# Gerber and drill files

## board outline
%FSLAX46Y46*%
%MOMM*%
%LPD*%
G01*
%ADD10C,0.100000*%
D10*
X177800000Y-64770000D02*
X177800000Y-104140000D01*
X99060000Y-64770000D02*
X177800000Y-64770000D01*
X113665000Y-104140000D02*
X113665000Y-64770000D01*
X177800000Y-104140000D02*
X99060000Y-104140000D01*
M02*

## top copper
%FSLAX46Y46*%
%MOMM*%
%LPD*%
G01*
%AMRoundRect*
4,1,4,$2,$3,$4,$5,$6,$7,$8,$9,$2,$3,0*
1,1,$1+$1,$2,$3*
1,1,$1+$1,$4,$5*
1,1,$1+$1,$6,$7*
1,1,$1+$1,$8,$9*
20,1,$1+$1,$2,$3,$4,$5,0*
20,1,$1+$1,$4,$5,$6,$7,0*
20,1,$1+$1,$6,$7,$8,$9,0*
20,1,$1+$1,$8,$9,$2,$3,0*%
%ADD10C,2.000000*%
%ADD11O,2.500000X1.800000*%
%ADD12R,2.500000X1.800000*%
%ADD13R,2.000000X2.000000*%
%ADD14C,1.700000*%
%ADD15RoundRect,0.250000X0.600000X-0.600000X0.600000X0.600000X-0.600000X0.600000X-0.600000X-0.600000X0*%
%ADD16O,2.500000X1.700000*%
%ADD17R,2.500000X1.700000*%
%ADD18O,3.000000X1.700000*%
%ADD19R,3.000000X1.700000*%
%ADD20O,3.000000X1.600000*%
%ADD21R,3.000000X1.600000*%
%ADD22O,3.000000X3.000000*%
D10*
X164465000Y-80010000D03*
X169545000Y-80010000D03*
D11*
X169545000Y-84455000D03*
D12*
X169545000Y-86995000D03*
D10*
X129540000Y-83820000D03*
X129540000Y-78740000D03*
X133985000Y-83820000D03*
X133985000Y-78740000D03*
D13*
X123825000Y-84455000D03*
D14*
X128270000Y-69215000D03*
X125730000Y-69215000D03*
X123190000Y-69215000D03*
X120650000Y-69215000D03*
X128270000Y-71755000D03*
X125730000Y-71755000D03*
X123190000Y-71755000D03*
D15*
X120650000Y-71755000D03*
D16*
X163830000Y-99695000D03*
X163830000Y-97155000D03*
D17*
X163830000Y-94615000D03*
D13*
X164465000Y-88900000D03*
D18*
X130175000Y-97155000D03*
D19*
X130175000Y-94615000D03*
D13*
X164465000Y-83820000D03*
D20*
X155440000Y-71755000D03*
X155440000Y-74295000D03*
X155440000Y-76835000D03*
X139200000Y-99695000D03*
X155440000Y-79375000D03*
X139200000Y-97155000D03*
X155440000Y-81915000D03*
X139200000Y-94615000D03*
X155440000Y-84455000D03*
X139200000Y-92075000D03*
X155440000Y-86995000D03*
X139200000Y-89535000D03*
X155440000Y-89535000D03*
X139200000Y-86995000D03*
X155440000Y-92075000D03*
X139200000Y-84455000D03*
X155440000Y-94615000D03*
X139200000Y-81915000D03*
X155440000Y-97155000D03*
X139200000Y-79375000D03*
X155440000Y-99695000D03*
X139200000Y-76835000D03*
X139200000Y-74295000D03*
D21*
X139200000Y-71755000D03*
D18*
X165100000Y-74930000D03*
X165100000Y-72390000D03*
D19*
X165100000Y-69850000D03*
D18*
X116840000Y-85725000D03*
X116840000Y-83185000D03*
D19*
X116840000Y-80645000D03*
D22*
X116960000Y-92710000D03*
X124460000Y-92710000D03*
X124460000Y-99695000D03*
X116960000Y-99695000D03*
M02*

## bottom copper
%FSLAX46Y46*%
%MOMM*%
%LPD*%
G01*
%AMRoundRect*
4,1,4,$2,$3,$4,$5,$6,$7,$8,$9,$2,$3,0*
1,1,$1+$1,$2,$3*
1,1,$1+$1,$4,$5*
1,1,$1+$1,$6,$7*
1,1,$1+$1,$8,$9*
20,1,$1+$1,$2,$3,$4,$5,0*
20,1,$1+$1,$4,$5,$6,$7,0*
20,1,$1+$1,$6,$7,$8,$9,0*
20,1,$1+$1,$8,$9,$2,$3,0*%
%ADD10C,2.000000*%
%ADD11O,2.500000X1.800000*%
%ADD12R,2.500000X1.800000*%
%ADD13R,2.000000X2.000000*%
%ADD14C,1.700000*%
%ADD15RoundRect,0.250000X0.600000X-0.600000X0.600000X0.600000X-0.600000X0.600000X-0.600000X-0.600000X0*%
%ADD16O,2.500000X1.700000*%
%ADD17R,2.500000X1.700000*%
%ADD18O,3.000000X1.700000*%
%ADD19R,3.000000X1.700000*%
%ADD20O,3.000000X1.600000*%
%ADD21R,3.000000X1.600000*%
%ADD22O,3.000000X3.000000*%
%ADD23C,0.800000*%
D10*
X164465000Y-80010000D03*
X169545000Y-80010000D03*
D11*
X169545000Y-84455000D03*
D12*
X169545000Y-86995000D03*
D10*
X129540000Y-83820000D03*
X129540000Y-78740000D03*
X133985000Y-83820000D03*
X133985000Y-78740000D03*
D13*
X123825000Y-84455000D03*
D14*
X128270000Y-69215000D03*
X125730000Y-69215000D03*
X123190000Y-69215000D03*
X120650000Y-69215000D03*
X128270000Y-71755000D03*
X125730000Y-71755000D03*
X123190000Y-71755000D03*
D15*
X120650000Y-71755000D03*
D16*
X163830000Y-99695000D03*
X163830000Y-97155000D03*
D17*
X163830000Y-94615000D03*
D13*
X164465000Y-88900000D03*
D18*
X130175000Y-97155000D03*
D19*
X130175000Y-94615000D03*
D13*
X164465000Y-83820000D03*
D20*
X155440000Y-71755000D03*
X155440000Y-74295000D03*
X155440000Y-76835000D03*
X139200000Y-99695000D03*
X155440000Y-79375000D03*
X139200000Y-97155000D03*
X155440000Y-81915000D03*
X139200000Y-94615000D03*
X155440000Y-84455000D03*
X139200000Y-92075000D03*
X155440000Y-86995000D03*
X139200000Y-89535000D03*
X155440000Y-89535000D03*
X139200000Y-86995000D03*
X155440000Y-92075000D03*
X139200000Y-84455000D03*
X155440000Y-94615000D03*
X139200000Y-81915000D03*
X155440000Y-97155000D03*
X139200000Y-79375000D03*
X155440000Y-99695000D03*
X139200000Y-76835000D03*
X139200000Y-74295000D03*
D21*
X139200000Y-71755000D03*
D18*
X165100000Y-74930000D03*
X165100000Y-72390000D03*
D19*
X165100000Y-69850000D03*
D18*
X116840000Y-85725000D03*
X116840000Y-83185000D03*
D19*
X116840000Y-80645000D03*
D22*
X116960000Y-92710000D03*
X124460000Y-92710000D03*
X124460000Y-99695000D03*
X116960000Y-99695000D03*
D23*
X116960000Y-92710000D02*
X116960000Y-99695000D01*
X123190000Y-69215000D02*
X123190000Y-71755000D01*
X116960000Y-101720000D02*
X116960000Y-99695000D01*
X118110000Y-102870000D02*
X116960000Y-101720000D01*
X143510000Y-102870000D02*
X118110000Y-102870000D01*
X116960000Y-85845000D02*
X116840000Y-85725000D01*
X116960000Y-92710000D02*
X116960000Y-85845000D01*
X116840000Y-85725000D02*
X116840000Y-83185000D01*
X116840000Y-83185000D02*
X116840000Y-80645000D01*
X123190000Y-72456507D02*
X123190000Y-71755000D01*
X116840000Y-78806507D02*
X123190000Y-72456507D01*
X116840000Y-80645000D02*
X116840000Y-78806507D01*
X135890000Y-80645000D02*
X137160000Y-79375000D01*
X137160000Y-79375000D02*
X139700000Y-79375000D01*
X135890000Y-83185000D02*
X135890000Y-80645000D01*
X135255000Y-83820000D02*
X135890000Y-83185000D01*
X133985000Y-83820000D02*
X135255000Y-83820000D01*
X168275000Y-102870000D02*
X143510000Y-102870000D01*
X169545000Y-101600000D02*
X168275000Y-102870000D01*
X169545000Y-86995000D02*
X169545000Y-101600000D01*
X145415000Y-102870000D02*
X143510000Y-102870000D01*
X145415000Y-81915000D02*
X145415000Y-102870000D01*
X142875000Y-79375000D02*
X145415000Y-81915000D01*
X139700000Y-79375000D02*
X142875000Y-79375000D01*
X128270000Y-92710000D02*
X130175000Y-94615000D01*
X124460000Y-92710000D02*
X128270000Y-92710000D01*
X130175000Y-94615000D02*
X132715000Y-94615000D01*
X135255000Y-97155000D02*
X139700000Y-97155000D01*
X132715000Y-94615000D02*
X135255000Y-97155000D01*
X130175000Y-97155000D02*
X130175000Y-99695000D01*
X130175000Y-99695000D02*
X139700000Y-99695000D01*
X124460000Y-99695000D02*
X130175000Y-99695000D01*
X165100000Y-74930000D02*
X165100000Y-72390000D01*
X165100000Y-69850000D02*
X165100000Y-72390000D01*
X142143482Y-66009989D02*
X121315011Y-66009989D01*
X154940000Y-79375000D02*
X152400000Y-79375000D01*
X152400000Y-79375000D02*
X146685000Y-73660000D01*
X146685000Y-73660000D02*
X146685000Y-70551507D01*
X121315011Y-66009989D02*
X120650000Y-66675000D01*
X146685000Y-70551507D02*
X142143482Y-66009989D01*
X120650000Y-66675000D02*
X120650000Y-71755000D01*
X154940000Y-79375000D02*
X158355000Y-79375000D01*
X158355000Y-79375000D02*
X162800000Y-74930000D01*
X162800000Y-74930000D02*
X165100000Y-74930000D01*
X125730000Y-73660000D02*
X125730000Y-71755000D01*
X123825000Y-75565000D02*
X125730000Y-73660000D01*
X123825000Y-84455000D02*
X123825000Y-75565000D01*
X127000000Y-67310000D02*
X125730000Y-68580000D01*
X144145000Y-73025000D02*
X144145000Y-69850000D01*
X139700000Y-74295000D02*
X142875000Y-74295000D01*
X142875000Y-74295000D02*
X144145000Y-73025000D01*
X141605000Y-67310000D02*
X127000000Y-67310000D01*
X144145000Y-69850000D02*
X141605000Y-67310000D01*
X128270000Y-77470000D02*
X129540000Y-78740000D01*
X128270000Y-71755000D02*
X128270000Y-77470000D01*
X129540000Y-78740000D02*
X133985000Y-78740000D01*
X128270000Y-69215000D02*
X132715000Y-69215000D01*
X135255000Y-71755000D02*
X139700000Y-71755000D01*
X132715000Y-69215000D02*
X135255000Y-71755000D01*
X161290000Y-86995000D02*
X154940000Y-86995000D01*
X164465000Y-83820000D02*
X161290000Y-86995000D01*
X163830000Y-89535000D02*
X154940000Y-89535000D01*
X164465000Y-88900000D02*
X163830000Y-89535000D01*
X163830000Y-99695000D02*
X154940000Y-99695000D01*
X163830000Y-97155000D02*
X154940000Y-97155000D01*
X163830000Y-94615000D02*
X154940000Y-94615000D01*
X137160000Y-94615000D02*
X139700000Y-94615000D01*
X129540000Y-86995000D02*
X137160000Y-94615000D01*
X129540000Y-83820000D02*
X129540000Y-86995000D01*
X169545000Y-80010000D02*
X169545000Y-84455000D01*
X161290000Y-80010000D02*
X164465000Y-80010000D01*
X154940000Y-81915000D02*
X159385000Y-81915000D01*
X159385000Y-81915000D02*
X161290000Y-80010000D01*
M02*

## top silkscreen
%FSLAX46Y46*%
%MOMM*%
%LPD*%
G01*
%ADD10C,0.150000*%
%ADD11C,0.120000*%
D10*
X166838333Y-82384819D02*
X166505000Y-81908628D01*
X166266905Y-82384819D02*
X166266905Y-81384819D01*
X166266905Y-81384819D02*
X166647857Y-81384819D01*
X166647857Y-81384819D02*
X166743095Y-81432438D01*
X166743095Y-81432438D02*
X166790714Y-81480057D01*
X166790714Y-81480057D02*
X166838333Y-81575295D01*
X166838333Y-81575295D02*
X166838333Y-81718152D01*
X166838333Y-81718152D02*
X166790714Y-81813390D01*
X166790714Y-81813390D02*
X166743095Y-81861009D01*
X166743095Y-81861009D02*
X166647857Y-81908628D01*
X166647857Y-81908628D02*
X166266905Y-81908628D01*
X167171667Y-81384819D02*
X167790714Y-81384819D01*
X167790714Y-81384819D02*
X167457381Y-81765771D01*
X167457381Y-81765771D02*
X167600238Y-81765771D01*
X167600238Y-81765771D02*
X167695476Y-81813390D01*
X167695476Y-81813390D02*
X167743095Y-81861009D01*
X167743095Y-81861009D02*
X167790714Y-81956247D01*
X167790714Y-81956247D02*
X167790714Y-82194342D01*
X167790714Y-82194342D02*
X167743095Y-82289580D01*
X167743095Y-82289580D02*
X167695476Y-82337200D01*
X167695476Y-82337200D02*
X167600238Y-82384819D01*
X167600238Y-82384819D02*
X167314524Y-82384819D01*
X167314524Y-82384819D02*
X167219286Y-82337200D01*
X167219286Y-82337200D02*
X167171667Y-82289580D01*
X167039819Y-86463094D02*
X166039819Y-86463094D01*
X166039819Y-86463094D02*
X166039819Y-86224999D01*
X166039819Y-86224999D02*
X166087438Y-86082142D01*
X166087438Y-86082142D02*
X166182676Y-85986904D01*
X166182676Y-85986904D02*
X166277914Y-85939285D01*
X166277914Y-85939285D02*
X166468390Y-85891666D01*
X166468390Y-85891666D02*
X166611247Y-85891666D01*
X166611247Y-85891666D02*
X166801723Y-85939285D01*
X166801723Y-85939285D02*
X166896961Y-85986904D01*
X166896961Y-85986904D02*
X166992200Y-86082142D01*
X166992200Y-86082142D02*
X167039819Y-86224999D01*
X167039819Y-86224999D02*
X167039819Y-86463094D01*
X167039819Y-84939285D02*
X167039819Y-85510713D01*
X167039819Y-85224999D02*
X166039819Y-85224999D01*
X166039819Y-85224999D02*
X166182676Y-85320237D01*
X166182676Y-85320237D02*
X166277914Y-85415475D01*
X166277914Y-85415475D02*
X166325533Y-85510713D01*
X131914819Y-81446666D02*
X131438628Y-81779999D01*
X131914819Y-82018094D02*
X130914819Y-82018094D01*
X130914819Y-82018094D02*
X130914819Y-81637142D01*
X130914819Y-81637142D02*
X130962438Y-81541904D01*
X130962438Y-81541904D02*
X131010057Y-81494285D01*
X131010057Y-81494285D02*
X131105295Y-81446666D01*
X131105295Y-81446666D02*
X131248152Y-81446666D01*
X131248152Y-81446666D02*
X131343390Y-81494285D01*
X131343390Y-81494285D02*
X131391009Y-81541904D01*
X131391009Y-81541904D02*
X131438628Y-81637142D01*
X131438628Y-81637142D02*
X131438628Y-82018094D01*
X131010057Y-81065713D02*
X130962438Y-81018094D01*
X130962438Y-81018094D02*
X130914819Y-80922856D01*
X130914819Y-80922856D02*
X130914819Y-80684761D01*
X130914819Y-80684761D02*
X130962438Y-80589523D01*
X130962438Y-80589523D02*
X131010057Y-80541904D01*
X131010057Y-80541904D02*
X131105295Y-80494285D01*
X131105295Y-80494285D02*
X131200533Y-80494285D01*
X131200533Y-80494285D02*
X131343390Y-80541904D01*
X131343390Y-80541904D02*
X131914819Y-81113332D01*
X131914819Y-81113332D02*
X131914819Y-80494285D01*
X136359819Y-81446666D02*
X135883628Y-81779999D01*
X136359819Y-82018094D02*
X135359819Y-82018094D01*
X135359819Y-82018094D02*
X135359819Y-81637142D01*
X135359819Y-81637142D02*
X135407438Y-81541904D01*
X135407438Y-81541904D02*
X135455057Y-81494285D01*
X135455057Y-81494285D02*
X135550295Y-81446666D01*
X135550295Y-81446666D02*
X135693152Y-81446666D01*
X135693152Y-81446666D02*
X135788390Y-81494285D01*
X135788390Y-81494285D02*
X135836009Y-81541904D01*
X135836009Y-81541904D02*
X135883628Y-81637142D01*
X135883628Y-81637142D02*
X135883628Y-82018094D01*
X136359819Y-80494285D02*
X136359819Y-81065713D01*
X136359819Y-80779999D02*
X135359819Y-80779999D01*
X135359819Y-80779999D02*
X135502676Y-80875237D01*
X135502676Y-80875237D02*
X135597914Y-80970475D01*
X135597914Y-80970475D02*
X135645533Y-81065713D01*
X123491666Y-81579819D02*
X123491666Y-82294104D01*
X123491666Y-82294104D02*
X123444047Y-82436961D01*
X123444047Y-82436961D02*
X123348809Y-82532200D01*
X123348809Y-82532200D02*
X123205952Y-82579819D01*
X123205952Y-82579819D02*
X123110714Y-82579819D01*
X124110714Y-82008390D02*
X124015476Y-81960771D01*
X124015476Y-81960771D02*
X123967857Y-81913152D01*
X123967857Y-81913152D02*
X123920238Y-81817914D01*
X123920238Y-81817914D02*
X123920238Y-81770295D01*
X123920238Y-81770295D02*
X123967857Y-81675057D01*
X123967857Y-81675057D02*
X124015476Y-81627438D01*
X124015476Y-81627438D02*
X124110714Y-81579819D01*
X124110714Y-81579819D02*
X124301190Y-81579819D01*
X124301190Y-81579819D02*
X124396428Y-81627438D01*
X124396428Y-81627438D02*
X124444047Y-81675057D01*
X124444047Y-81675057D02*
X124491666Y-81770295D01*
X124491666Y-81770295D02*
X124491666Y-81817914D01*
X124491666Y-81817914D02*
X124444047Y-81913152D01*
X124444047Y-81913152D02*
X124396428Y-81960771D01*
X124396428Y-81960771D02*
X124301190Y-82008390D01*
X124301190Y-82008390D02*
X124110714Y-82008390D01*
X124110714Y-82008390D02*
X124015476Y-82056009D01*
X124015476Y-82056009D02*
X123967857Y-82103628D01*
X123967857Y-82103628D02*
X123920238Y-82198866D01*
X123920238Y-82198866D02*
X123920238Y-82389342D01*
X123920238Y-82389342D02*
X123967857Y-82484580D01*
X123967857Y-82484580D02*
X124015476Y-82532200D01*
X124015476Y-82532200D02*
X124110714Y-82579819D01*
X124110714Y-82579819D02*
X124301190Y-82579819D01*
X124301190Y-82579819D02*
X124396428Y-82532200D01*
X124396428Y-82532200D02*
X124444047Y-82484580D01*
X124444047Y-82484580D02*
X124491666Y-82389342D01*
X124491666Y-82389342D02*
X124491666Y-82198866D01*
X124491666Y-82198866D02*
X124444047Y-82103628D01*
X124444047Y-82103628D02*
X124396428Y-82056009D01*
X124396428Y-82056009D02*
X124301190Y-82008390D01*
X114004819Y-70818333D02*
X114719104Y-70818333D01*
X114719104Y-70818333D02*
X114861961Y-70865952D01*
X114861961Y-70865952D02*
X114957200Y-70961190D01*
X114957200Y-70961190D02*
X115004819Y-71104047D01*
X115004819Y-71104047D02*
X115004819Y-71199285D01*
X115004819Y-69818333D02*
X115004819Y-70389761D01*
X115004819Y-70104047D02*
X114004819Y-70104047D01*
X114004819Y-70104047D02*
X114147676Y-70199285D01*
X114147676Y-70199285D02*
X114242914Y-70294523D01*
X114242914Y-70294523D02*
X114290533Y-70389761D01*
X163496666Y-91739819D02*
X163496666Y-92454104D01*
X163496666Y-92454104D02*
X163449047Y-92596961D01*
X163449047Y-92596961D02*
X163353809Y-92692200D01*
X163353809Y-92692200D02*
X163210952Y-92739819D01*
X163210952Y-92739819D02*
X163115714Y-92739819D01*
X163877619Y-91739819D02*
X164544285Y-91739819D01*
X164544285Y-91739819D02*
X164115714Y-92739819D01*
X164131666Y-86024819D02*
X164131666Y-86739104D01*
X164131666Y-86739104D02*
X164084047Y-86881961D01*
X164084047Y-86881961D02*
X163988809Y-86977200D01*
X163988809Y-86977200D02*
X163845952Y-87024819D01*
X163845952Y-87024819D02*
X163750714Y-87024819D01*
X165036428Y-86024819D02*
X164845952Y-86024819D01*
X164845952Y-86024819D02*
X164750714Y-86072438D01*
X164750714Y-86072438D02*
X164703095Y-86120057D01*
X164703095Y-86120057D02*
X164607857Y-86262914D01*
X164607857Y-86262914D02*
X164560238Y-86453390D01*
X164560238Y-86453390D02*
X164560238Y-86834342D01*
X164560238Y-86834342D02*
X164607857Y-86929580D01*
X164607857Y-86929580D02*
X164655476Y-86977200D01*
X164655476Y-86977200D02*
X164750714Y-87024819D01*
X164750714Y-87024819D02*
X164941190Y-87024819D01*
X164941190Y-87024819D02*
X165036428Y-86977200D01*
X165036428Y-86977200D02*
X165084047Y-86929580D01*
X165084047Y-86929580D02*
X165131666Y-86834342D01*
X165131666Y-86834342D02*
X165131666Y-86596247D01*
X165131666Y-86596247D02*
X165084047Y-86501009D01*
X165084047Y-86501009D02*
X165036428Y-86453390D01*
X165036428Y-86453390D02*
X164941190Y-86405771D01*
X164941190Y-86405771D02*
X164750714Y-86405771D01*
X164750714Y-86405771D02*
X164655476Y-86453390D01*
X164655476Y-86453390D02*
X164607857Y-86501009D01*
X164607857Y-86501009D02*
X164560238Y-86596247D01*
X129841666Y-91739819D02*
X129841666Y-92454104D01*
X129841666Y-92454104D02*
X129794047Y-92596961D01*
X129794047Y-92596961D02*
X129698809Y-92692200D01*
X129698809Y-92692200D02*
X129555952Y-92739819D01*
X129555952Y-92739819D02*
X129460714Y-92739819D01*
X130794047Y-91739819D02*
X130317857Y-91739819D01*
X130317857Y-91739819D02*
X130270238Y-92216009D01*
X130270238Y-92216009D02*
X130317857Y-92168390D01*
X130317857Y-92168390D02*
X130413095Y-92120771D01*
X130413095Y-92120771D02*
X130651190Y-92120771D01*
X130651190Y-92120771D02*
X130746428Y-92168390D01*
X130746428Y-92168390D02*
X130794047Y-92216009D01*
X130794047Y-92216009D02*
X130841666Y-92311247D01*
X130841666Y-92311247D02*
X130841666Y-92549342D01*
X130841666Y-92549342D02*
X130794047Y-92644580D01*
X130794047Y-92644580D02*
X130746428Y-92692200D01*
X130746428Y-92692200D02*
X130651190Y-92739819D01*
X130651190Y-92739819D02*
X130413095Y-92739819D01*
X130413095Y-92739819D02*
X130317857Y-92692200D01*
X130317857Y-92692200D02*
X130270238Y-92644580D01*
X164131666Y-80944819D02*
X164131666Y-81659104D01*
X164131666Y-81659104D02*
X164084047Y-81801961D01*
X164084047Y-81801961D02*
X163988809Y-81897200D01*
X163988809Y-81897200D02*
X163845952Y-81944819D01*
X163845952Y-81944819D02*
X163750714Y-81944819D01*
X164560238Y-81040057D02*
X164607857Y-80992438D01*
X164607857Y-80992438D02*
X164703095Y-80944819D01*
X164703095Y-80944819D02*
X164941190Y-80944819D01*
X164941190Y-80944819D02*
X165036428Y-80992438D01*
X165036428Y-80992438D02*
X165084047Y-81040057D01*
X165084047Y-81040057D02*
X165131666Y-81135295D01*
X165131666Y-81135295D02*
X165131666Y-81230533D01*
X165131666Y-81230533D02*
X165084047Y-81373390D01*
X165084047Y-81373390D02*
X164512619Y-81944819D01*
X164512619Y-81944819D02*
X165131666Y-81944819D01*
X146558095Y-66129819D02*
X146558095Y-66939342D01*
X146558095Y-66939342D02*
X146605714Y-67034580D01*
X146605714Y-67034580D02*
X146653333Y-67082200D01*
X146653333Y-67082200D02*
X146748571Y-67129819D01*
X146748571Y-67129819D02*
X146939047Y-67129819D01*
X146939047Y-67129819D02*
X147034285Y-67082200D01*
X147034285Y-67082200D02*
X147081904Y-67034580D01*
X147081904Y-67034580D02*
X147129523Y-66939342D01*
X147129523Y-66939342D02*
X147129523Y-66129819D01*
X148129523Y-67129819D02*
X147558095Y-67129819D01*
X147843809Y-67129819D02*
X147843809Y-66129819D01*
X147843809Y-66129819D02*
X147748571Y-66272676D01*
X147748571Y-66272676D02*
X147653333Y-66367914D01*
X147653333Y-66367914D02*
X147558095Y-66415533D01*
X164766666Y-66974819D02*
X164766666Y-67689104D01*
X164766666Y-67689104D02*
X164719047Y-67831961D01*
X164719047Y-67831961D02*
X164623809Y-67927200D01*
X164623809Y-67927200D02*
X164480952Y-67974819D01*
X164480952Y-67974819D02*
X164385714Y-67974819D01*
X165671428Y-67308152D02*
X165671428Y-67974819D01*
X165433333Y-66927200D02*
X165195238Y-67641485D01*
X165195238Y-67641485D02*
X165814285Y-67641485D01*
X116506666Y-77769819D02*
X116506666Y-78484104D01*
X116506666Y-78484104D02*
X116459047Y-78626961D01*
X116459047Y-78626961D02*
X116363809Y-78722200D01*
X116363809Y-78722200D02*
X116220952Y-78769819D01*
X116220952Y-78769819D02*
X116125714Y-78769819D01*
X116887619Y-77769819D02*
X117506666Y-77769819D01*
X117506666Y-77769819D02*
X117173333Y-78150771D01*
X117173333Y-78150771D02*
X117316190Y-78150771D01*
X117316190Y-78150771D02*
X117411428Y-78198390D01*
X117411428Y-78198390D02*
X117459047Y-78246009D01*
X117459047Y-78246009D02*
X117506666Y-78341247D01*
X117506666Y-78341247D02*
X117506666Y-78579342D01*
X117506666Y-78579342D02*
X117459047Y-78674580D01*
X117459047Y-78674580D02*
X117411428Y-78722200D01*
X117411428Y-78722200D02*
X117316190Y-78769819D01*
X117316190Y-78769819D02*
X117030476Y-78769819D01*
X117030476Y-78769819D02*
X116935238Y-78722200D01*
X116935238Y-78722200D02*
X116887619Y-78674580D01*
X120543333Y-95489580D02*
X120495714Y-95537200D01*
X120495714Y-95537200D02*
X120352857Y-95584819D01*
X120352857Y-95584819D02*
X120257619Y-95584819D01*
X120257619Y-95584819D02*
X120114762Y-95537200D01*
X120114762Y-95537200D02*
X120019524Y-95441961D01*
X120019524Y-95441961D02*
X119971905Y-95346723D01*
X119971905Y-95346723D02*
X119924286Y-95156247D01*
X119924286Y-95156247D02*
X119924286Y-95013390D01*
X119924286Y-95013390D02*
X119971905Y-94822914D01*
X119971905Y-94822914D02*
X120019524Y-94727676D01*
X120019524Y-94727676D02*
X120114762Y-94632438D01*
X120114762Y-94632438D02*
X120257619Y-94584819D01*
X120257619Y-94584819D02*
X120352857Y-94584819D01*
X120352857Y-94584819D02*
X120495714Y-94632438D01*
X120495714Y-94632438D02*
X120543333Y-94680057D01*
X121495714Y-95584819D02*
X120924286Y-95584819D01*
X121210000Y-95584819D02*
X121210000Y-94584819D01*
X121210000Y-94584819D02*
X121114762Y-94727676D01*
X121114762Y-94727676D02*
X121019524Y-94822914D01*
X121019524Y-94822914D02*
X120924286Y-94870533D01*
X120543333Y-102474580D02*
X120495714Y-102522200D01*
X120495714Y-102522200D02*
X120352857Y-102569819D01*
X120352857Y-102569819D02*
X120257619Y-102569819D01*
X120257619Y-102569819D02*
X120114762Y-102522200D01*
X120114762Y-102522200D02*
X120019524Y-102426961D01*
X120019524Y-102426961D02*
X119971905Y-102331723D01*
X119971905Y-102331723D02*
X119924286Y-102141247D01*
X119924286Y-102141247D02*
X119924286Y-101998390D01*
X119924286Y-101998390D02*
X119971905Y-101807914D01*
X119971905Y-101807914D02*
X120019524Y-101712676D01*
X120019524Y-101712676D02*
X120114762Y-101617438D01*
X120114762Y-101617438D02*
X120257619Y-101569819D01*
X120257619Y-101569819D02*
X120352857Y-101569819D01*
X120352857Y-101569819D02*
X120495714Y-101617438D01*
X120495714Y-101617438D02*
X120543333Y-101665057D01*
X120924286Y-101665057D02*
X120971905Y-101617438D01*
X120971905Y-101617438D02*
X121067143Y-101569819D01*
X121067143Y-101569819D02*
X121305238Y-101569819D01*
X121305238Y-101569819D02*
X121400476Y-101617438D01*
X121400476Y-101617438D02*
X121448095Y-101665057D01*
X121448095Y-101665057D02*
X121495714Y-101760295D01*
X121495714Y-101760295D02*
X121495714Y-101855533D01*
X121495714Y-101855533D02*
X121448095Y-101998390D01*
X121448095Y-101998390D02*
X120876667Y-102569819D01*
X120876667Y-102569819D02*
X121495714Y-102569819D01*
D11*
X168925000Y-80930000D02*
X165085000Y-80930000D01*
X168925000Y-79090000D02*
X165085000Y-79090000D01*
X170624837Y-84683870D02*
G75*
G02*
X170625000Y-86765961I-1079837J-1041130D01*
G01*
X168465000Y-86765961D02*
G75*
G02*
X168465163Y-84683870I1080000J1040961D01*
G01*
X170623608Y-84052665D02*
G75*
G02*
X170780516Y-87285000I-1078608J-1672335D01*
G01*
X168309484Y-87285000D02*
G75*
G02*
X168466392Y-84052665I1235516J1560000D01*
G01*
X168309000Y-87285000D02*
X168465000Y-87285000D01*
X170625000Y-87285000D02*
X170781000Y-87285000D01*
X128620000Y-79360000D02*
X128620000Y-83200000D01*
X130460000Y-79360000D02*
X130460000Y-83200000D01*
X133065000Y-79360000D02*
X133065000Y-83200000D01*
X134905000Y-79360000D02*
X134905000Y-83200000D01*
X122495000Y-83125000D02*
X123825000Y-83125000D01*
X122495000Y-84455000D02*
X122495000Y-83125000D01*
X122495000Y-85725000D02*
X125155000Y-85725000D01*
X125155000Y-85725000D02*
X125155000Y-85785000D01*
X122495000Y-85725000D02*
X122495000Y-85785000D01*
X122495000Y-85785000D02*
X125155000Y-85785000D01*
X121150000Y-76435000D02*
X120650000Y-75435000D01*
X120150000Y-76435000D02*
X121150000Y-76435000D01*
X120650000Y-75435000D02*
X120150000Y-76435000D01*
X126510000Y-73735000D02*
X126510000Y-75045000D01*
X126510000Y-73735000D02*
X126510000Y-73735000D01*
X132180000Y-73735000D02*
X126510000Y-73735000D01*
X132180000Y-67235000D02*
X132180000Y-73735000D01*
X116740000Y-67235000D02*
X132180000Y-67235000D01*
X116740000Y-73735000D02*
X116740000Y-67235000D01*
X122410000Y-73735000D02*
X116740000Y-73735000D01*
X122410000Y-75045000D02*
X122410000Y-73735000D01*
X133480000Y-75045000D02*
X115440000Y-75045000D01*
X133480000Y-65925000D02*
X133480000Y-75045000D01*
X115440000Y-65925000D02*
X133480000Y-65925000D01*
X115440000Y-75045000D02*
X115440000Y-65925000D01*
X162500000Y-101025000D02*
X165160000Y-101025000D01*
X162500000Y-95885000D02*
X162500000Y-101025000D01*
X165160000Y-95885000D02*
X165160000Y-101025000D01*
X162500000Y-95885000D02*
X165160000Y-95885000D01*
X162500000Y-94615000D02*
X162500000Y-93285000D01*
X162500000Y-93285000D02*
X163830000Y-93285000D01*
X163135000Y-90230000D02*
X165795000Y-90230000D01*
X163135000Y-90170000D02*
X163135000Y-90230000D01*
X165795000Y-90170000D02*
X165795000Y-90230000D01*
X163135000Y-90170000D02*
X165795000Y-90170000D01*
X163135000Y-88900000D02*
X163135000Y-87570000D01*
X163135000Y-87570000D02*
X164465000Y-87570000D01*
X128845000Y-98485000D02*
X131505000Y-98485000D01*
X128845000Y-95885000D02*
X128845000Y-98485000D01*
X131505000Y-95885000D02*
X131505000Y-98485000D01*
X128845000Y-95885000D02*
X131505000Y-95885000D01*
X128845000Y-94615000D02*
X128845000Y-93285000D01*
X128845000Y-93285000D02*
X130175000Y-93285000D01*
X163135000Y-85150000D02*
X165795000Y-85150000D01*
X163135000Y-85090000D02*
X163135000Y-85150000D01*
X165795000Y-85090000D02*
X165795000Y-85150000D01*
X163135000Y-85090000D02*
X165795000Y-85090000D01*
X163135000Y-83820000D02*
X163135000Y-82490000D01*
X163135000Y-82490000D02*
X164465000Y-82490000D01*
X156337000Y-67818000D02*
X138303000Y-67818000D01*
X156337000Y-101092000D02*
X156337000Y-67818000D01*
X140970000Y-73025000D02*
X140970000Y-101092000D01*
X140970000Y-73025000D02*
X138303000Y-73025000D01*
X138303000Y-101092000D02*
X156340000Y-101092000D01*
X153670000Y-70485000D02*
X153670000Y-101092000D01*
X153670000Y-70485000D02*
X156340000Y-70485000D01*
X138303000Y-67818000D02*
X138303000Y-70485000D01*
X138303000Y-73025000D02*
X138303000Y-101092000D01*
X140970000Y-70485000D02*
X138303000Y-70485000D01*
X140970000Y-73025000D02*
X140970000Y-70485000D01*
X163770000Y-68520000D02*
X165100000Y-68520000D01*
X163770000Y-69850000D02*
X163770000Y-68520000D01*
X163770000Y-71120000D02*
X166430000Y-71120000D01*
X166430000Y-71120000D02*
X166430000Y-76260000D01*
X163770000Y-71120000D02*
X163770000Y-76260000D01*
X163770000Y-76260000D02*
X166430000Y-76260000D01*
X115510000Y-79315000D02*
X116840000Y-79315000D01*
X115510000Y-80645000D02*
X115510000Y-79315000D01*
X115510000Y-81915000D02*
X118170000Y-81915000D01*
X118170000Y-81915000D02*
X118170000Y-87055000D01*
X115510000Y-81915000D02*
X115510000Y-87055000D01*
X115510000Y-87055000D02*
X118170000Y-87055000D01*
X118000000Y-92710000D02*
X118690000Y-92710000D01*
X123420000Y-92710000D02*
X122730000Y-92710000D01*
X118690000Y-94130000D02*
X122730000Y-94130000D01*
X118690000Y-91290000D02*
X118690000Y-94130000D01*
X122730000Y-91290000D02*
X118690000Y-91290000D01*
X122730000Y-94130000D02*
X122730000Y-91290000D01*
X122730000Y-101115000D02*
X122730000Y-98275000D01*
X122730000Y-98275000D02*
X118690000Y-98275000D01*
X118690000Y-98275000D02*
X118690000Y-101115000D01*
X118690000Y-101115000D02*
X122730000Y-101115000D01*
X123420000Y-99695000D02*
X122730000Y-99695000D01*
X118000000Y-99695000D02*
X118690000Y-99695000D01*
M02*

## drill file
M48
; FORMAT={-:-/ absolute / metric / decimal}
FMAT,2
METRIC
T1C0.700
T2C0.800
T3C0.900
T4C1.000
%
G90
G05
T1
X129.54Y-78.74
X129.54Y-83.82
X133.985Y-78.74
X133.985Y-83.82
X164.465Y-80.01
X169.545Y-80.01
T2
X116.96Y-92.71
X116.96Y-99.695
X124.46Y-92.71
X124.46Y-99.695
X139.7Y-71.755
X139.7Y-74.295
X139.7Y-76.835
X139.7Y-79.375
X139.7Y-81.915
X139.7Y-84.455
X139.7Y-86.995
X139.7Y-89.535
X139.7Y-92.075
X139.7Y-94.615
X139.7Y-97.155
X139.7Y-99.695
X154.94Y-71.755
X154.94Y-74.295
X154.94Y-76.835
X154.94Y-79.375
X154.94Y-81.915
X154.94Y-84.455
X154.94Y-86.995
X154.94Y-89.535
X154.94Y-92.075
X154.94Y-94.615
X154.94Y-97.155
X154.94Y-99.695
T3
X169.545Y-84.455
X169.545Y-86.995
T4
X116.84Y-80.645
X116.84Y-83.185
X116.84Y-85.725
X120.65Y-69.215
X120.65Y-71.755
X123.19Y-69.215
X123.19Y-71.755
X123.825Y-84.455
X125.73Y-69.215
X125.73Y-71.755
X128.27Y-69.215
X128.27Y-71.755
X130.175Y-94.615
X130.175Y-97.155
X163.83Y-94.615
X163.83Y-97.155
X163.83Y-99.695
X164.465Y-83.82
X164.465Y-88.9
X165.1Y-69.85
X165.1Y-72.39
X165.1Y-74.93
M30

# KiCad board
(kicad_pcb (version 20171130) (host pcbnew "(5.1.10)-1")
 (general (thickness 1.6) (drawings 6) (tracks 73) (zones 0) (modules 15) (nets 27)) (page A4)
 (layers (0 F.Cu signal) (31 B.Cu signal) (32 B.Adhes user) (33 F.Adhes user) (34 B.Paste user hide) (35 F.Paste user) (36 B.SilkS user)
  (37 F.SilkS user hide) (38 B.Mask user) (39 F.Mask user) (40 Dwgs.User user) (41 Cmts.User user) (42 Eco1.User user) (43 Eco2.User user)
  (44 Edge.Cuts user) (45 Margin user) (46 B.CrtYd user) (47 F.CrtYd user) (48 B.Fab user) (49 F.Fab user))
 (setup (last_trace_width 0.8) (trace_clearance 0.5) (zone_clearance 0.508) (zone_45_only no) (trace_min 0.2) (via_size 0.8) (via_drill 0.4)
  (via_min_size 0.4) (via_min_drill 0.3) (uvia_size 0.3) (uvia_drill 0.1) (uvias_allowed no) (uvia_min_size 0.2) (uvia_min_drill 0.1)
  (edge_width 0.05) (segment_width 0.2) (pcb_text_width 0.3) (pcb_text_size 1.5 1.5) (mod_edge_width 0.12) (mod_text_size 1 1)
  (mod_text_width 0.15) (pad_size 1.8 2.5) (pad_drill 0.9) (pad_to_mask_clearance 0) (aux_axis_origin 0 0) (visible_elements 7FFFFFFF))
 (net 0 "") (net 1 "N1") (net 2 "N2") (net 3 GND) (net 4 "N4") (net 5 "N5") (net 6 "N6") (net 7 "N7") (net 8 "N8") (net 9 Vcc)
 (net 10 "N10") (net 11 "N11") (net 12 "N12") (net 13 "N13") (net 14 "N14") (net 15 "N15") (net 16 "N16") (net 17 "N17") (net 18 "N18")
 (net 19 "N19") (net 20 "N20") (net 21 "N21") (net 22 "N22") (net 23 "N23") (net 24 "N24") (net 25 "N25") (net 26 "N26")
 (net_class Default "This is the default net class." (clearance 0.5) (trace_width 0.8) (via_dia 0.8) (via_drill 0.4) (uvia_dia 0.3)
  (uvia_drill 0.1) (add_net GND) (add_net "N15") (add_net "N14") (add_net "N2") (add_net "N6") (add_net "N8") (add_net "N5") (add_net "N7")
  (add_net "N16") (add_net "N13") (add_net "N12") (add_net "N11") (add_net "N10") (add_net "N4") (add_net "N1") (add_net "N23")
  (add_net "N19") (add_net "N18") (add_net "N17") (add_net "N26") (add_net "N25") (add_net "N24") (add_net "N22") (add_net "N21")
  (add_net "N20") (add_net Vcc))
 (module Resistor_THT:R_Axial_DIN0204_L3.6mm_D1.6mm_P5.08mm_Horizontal (layer F.Cu) (at 169.545 80.01 180)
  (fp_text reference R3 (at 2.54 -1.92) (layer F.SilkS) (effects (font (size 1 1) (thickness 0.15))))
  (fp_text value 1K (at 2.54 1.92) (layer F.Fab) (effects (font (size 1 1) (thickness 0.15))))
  (fp_line (start 0.62 -0.92) (end 4.46 -0.92) (layer F.SilkS) (width 0.12))
  (fp_line (start 0.62 0.92) (end 4.46 0.92) (layer F.SilkS) (width 0.12))
  (pad 2 thru_hole circle (at 5.08 0 180) (size 2 2) (drill 0.7) (layers *.Cu *.Mask) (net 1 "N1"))
  (pad 1 thru_hole circle (at 0 0 180) (size 2 2) (drill 0.7) (layers *.Cu *.Mask) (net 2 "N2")))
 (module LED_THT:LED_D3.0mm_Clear (layer F.Cu) (at 169.545 86.995 90)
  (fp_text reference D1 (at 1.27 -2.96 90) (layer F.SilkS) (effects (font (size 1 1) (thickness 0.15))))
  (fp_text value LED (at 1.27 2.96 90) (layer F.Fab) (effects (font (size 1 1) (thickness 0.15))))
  (fp_arc (start 1.27 0) (end 0.229039 1.08) (angle -87.9) (layer F.SilkS) (width 0.12))
  (fp_arc (start 1.27 0) (end 0.229039 -1.08) (angle 87.9) (layer F.SilkS) (width 0.12))
  (fp_arc (start 1.27 0) (end -0.29 1.235516) (angle -108.8) (layer F.SilkS) (width 0.12))
  (fp_arc (start 1.27 0) (end -0.29 -1.235516) (angle 108.8) (layer F.SilkS) (width 0.12))
  (fp_line (start -0.29 -1.236) (end -0.29 -1.08) (layer F.SilkS) (width 0.12))
  (fp_line (start -0.29 1.08) (end -0.29 1.236) (layer F.SilkS) (width 0.12))
  (pad 2 thru_hole oval (at 2.54 0 90) (size 1.8 2.5) (drill 0.9) (layers *.Cu *.Mask) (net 2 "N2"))
  (pad 1 thru_hole rect (at 0 0 90) (size 1.8 2.5) (drill 0.9) (layers *.Cu *.Mask) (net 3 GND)))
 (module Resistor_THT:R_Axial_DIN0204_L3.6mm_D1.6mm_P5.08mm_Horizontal (layer F.Cu) (at 129.54 78.74 270)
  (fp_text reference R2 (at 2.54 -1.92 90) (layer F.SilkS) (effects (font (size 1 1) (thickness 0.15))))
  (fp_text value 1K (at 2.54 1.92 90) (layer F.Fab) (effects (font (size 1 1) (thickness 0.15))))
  (fp_line (start 0.62 0.92) (end 4.46 0.92) (layer F.SilkS) (width 0.12))
  (fp_line (start 0.62 -0.92) (end 4.46 -0.92) (layer F.SilkS) (width 0.12))
  (pad 2 thru_hole circle (at 5.08 0 270) (size 2 2) (drill 0.7) (layers *.Cu *.Mask) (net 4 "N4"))
  (pad 1 thru_hole circle (at 0 0 270) (size 2 2) (drill 0.7) (layers *.Cu *.Mask) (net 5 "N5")))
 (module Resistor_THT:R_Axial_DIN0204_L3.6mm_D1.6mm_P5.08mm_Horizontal (layer F.Cu) (at 133.985 78.74 270)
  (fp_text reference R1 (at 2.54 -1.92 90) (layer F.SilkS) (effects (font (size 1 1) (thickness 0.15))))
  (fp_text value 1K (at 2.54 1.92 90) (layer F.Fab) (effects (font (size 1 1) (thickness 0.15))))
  (fp_line (start 0.62 0.92) (end 4.46 0.92) (layer F.SilkS) (width 0.12))
  (fp_line (start 0.62 -0.92) (end 4.46 -0.92) (layer F.SilkS) (width 0.12))
  (pad 2 thru_hole circle (at 5.08 0 270) (size 2 2) (drill 0.7) (layers *.Cu *.Mask) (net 3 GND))
  (pad 1 thru_hole circle (at 0 0 270) (size 2 2) (drill 0.7) (layers *.Cu *.Mask) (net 5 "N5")))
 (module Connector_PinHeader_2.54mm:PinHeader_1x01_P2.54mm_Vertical (layer F.Cu) (at 123.825 84.455)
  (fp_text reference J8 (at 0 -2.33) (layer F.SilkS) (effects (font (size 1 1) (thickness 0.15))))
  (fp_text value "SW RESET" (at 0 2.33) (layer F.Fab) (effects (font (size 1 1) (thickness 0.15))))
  (fp_line (start -1.33 -1.33) (end 0 -1.33) (layer F.SilkS) (width 0.12))
  (fp_line (start -1.33 0) (end -1.33 -1.33) (layer F.SilkS) (width 0.12))
  (fp_line (start -1.33 1.27) (end 1.33 1.27) (layer F.SilkS) (width 0.12))
  (fp_line (start 1.33 1.27) (end 1.33 1.33) (layer F.SilkS) (width 0.12))
  (fp_line (start -1.33 1.27) (end -1.33 1.33) (layer F.SilkS) (width 0.12))
  (fp_line (start -1.33 1.33) (end 1.33 1.33) (layer F.SilkS) (width 0.12))
  (pad 1 thru_hole rect (at 0 0) (size 2 2) (drill 1) (layers *.Cu *.Mask) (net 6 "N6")))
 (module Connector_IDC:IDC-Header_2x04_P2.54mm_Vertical (layer F.Cu) (at 120.65 71.755 90)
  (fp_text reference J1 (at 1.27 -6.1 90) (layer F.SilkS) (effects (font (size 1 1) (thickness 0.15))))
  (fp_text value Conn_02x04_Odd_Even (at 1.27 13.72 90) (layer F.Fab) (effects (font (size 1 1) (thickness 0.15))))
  (fp_line (start -4.68 0.5) (end -3.68 0) (layer F.SilkS) (width 0.12))
  (fp_line (start -4.68 -0.5) (end -4.68 0.5) (layer F.SilkS) (width 0.12))
  (fp_line (start -3.68 0) (end -4.68 -0.5) (layer F.SilkS) (width 0.12))
  (fp_line (start -1.98 5.86) (end -3.29 5.86) (layer F.SilkS) (width 0.12))
  (fp_line (start -1.98 5.86) (end -1.98 5.86) (layer F.SilkS) (width 0.12))
  (fp_line (start -1.98 11.53) (end -1.98 5.86) (layer F.SilkS) (width 0.12))
  (fp_line (start 4.52 11.53) (end -1.98 11.53) (layer F.SilkS) (width 0.12))
  (fp_line (start 4.52 -3.91) (end 4.52 11.53) (layer F.SilkS) (width 0.12))
  (fp_line (start -1.98 -3.91) (end 4.52 -3.91) (layer F.SilkS) (width 0.12))
  (fp_line (start -1.98 1.76) (end -1.98 -3.91) (layer F.SilkS) (width 0.12))
  (fp_line (start -3.29 1.76) (end -1.98 1.76) (layer F.SilkS) (width 0.12))
  (fp_line (start -3.29 12.83) (end -3.29 -5.21) (layer F.SilkS) (width 0.12))
  (fp_line (start 5.83 12.83) (end -3.29 12.83) (layer F.SilkS) (width 0.12))
  (fp_line (start 5.83 -5.21) (end 5.83 12.83) (layer F.SilkS) (width 0.12))
  (fp_line (start -3.29 -5.21) (end 5.83 -5.21) (layer F.SilkS) (width 0.12))
  (pad 8 thru_hole circle (at 2.54 7.62 90) (size 1.7 1.7) (drill 1) (layers *.Cu *.Mask) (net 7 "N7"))
  (pad 6 thru_hole circle (at 2.54 5.08 90) (size 1.7 1.7) (drill 1) (layers *.Cu *.Mask) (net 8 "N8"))
  (pad 4 thru_hole circle (at 2.54 2.54 90) (size 1.7 1.7) (drill 1) (layers *.Cu *.Mask) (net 3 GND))
  (pad 2 thru_hole circle (at 2.54 0 90) (size 1.7 1.7) (drill 1) (layers *.Cu *.Mask) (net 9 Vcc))
  (pad 7 thru_hole circle (at 0 7.62 90) (size 1.7 1.7) (drill 1) (layers *.Cu *.Mask) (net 5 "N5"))
  (pad 5 thru_hole circle (at 0 5.08 90) (size 1.7 1.7) (drill 1) (layers *.Cu *.Mask) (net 6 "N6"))
  (pad 3 thru_hole circle (at 0 2.54 90) (size 1.7 1.7) (drill 1) (layers *.Cu *.Mask) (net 3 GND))
  (pad 1 thru_hole roundrect (at 0 0 90) (size 1.7 1.7) (drill 1) (layers *.Cu *.Mask) (roundrect_rratio 0.147059) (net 9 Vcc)))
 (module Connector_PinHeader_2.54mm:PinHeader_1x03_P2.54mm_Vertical (layer F.Cu) (at 163.83 94.615)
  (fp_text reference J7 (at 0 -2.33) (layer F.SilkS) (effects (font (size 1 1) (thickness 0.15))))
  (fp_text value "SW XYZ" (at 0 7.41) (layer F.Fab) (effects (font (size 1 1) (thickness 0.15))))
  (fp_line (start -1.33 6.41) (end 1.33 6.41) (layer F.SilkS) (width 0.12))
  (fp_line (start -1.33 1.27) (end -1.33 6.41) (layer F.SilkS) (width 0.12))
  (fp_line (start 1.33 1.27) (end 1.33 6.41) (layer F.SilkS) (width 0.12))
  (fp_line (start -1.33 1.27) (end 1.33 1.27) (layer F.SilkS) (width 0.12))
  (fp_line (start -1.33 0) (end -1.33 -1.33) (layer F.SilkS) (width 0.12))
  (fp_line (start -1.33 -1.33) (end 0 -1.33) (layer F.SilkS) (width 0.12))
  (pad 3 thru_hole oval (at 0 5.08) (size 2.5 1.7) (drill 1) (layers *.Cu *.Mask) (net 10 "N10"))
  (pad 2 thru_hole oval (at 0 2.54) (size 2.5 1.7) (drill 1) (layers *.Cu *.Mask) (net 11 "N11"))
  (pad 1 thru_hole rect (at 0 0) (size 2.5 1.7) (drill 1) (layers *.Cu *.Mask) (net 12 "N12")))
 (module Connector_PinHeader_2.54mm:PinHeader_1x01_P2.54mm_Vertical (layer F.Cu) (at 164.465 88.9)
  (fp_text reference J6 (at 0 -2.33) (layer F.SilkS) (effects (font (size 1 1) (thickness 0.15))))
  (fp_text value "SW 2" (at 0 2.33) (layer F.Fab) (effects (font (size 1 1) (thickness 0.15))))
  (fp_line (start -1.33 1.33) (end 1.33 1.33) (layer F.SilkS) (width 0.12))
  (fp_line (start -1.33 1.27) (end -1.33 1.33) (layer F.SilkS) (width 0.12))
  (fp_line (start 1.33 1.27) (end 1.33 1.33) (layer F.SilkS) (width 0.12))
  (fp_line (start -1.33 1.27) (end 1.33 1.27) (layer F.SilkS) (width 0.12))
  (fp_line (start -1.33 0) (end -1.33 -1.33) (layer F.SilkS) (width 0.12))
  (fp_line (start -1.33 -1.33) (end 0 -1.33) (layer F.SilkS) (width 0.12))
  (pad 1 thru_hole rect (at 0 0) (size 2 2) (drill 1) (layers *.Cu *.Mask) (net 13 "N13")))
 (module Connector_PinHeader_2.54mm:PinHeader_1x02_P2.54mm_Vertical (layer F.Cu) (at 130.175 94.615)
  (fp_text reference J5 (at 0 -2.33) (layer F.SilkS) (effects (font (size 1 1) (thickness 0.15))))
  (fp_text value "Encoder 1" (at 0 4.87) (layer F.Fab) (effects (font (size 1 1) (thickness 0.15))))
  (fp_line (start -1.33 3.87) (end 1.33 3.87) (layer F.SilkS) (width 0.12))
  (fp_line (start -1.33 1.27) (end -1.33 3.87) (layer F.SilkS) (width 0.12))
  (fp_line (start 1.33 1.27) (end 1.33 3.87) (layer F.SilkS) (width 0.12))
  (fp_line (start -1.33 1.27) (end 1.33 1.27) (layer F.SilkS) (width 0.12))
  (fp_line (start -1.33 0) (end -1.33 -1.33) (layer F.SilkS) (width 0.12))
  (fp_line (start -1.33 -1.33) (end 0 -1.33) (layer F.SilkS) (width 0.12))
  (pad 2 thru_hole oval (at 0 2.54) (size 3 1.7) (drill 1) (layers *.Cu *.Mask) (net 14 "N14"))
  (pad 1 thru_hole rect (at 0 0) (size 3 1.7) (drill 1) (layers *.Cu *.Mask) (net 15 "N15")))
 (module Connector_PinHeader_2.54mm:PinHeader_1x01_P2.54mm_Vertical (layer F.Cu) (at 164.465 83.82)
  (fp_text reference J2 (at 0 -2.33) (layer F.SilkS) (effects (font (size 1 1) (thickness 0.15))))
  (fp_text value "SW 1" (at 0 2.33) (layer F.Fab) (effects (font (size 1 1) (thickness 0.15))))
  (fp_line (start -1.33 1.33) (end 1.33 1.33) (layer F.SilkS) (width 0.12))
  (fp_line (start -1.33 1.27) (end -1.33 1.33) (layer F.SilkS) (width 0.12))
  (fp_line (start 1.33 1.27) (end 1.33 1.33) (layer F.SilkS) (width 0.12))
  (fp_line (start -1.33 1.27) (end 1.33 1.27) (layer F.SilkS) (width 0.12))
  (fp_line (start -1.33 0) (end -1.33 -1.33) (layer F.SilkS) (width 0.12))
  (fp_line (start -1.33 -1.33) (end 0 -1.33) (layer F.SilkS) (width 0.12))
  (pad 1 thru_hole rect (at 0 0) (size 2 2) (drill 1) (layers *.Cu *.Mask) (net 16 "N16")))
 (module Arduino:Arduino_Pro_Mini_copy (layer F.Cu) (at 139.7 71.755)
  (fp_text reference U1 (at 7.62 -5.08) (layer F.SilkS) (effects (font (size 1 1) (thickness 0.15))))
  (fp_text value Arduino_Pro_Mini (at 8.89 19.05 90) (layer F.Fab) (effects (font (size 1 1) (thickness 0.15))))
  (fp_line (start 16.637 -3.937) (end -1.397 -3.937) (layer F.SilkS) (width 0.12))
  (fp_line (start 16.637 29.337) (end 16.637 -3.937) (layer F.SilkS) (width 0.12))
  (fp_line (start 1.27 1.27) (end 1.27 29.337) (layer F.SilkS) (width 0.12))
  (fp_line (start 1.27 1.27) (end -1.397 1.27) (layer F.SilkS) (width 0.12))
  (fp_line (start -1.397 29.337) (end 16.64 29.337) (layer F.SilkS) (width 0.12))
  (fp_line (start 13.97 -1.27) (end 13.97 29.337) (layer F.SilkS) (width 0.12))
  (fp_line (start 13.97 -1.27) (end 16.64 -1.27) (layer F.SilkS) (width 0.12))
  (fp_line (start -1.397 -3.937) (end -1.397 -1.27) (layer F.SilkS) (width 0.12))
  (fp_line (start -1.397 1.27) (end -1.397 29.337) (layer F.SilkS) (width 0.12))
  (fp_line (start 1.27 -1.27) (end -1.397 -1.27) (layer F.SilkS) (width 0.12))
  (fp_line (start 1.27 1.27) (end 1.27 -1.27) (layer F.SilkS) (width 0.12))
  (pad 24 thru_hole oval (at 15.24 0) (size 3 1.6) (drill 0.8 (offset 0.5 0)) (layers *.Cu *.Mask) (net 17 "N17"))
  (pad 23 thru_hole oval (at 15.24 2.54) (size 3 1.6) (drill 0.8 (offset 0.5 0)) (layers *.Cu *.Mask) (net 3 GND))
  (pad 22 thru_hole oval (at 15.24 5.08) (size 3 1.6) (drill 0.8 (offset 0.5 0)) (layers *.Cu *.Mask) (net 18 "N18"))
  (pad 12 thru_hole oval (at 0 27.94) (size 3 1.6) (drill 0.8 (offset -0.5 0)) (layers *.Cu *.Mask) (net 14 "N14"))
  (pad 21 thru_hole oval (at 15.24 7.62) (size 3 1.6) (drill 0.8 (offset 0.5 0)) (layers *.Cu *.Mask) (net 9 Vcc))
  (pad 11 thru_hole oval (at 0 25.4) (size 3 1.6) (drill 0.8 (offset -0.5 0)) (layers *.Cu *.Mask) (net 15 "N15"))
  (pad 20 thru_hole oval (at 15.24 10.16) (size 3 1.6) (drill 0.8 (offset 0.5 0)) (layers *.Cu *.Mask) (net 1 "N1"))
  (pad 10 thru_hole oval (at 0 22.86) (size 3 1.6) (drill 0.8 (offset -0.5 0)) (layers *.Cu *.Mask) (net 4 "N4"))
  (pad 19 thru_hole oval (at 15.24 12.7) (size 3 1.6) (drill 0.8 (offset 0.5 0)) (layers *.Cu *.Mask) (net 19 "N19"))
  (pad 9 thru_hole oval (at 0 20.32) (size 3 1.6) (drill 0.8 (offset -0.5 0)) (layers *.Cu *.Mask) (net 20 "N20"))
  (pad 18 thru_hole oval (at 15.24 15.24) (size 3 1.6) (drill 0.8 (offset 0.5 0)) (layers *.Cu *.Mask) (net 16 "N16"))
  (pad 8 thru_hole oval (at 0 17.78) (size 3 1.6) (drill 0.8 (offset -0.5 0)) (layers *.Cu *.Mask) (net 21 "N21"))
  (pad 17 thru_hole oval (at 15.24 17.78) (size 3 1.6) (drill 0.8 (offset 0.5 0)) (layers *.Cu *.Mask) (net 13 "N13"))
  (pad 7 thru_hole oval (at 0 15.24) (size 3 1.6) (drill 0.8 (offset -0.5 0)) (layers *.Cu *.Mask) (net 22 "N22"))
  (pad 16 thru_hole oval (at 15.24 20.32) (size 3 1.6) (drill 0.8 (offset 0.5 0)) (layers *.Cu *.Mask) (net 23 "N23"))
  (pad 6 thru_hole oval (at 0 12.7) (size 3 1.6) (drill 0.8 (offset -0.5 0)) (layers *.Cu *.Mask) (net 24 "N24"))
  (pad 15 thru_hole oval (at 15.24 22.86) (size 3 1.6) (drill 0.8 (offset 0.5 0)) (layers *.Cu *.Mask) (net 12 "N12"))
  (pad 5 thru_hole oval (at 0 10.16) (size 3 1.6) (drill 0.8 (offset -0.5 0)) (layers *.Cu *.Mask) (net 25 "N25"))
  (pad 14 thru_hole oval (at 15.24 25.4) (size 3 1.6) (drill 0.8 (offset 0.5 0)) (layers *.Cu *.Mask) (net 11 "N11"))
  (pad 4 thru_hole oval (at 0 7.62) (size 3 1.6) (drill 0.8 (offset -0.5 0)) (layers *.Cu *.Mask) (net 3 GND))
  (pad 13 thru_hole oval (at 15.24 27.94) (size 3 1.6) (drill 0.8 (offset 0.5 0)) (layers *.Cu *.Mask) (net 10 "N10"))
  (pad 3 thru_hole oval (at 0 5.08) (size 3 1.6) (drill 0.8 (offset -0.5 0)) (layers *.Cu *.Mask) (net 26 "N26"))
  (pad 2 thru_hole oval (at 0 2.54) (size 3 1.6) (drill 0.8 (offset -0.5 0)) (layers *.Cu *.Mask) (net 8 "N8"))
  (pad 1 thru_hole rect (at 0 0) (size 3 1.6) (drill 0.8 (offset -0.5 0)) (layers *.Cu *.Mask) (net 7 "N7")))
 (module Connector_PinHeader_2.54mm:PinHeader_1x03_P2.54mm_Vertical (layer F.Cu) (at 165.1 69.85)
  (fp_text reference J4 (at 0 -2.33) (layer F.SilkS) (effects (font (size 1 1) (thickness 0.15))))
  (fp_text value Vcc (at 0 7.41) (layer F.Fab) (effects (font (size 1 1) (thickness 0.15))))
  (fp_line (start -1.33 -1.33) (end 0 -1.33) (layer F.SilkS) (width 0.12))
  (fp_line (start -1.33 0) (end -1.33 -1.33) (layer F.SilkS) (width 0.12))
  (fp_line (start -1.33 1.27) (end 1.33 1.27) (layer F.SilkS) (width 0.12))
  (fp_line (start 1.33 1.27) (end 1.33 6.41) (layer F.SilkS) (width 0.12))
  (fp_line (start -1.33 1.27) (end -1.33 6.41) (layer F.SilkS) (width 0.12))
  (fp_line (start -1.33 6.41) (end 1.33 6.41) (layer F.SilkS) (width 0.12))
  (pad 3 thru_hole oval (at 0 5.08) (size 3 1.7) (drill 1) (layers *.Cu *.Mask) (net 9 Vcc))
  (pad 2 thru_hole oval (at 0 2.54) (size 3 1.7) (drill 1) (layers *.Cu *.Mask) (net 9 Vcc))
  (pad 1 thru_hole rect (at 0 0) (size 3 1.7) (drill 1) (layers *.Cu *.Mask) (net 9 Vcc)))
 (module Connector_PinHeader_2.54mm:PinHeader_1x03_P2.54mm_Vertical (layer F.Cu) (at 116.84 80.645)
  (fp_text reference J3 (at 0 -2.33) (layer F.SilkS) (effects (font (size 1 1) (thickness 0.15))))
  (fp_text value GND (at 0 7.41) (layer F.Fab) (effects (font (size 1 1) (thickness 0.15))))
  (fp_line (start -1.33 -1.33) (end 0 -1.33) (layer F.SilkS) (width 0.12))
  (fp_line (start -1.33 0) (end -1.33 -1.33) (layer F.SilkS) (width 0.12))
  (fp_line (start -1.33 1.27) (end 1.33 1.27) (layer F.SilkS) (width 0.12))
  (fp_line (start 1.33 1.27) (end 1.33 6.41) (layer F.SilkS) (width 0.12))
  (fp_line (start -1.33 1.27) (end -1.33 6.41) (layer F.SilkS) (width 0.12))
  (fp_line (start -1.33 6.41) (end 1.33 6.41) (layer F.SilkS) (width 0.12))
  (pad 3 thru_hole oval (at 0 5.08) (size 3 1.7) (drill 1) (layers *.Cu *.Mask) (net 3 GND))
  (pad 2 thru_hole oval (at 0 2.54) (size 3 1.7) (drill 1) (layers *.Cu *.Mask) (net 3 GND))
  (pad 1 thru_hole rect (at 0 0) (size 3 1.7) (drill 1) (layers *.Cu *.Mask) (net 3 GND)))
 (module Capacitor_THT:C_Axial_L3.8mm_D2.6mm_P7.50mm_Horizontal (layer F.Cu) (at 124.46 92.71 180)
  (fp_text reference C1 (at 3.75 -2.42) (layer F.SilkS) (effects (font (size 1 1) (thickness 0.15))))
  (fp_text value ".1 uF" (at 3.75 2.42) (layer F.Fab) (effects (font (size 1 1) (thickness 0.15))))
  (fp_line (start 6.46 0) (end 5.77 0) (layer F.SilkS) (width 0.12))
  (fp_line (start 1.04 0) (end 1.73 0) (layer F.SilkS) (width 0.12))
  (fp_line (start 5.77 -1.42) (end 1.73 -1.42) (layer F.SilkS) (width 0.12))
  (fp_line (start 5.77 1.42) (end 5.77 -1.42) (layer F.SilkS) (width 0.12))
  (fp_line (start 1.73 1.42) (end 5.77 1.42) (layer F.SilkS) (width 0.12))
  (fp_line (start 1.73 -1.42) (end 1.73 1.42) (layer F.SilkS) (width 0.12))
  (pad 2 thru_hole oval (at 7.5 0 180) (size 3 3) (drill 0.8) (layers *.Cu *.Mask) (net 3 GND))
  (pad 1 thru_hole oval (at 0 0 180) (size 3 3) (drill 0.8) (layers *.Cu *.Mask) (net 15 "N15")))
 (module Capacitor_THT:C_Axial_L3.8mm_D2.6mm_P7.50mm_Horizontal (layer F.Cu) (at 124.46 99.695 180)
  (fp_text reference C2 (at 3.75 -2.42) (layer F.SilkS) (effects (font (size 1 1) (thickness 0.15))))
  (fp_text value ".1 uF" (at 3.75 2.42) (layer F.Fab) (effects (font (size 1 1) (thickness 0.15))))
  (fp_line (start 1.73 -1.42) (end 1.73 1.42) (layer F.SilkS) (width 0.12))
  (fp_line (start 1.73 1.42) (end 5.77 1.42) (layer F.SilkS) (width 0.12))
  (fp_line (start 5.77 1.42) (end 5.77 -1.42) (layer F.SilkS) (width 0.12))
  (fp_line (start 5.77 -1.42) (end 1.73 -1.42) (layer F.SilkS) (width 0.12))
  (fp_line (start 1.04 0) (end 1.73 0) (layer F.SilkS) (width 0.12))
  (fp_line (start 6.46 0) (end 5.77 0) (layer F.SilkS) (width 0.12))
  (pad 1 thru_hole oval (at 0 0 180) (size 3 3) (drill 0.8) (layers *.Cu *.Mask) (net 14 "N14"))
  (pad 2 thru_hole oval (at 7.5 0 180) (size 3 3) (drill 0.8) (layers *.Cu *.Mask) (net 3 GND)))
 (gr_line (start 177.8 64.77) (end 177.8 104.14) (layer Edge.Cuts) (width 0.1))
 (gr_line (start 99.06 64.77) (end 177.8 64.77) (layer Edge.Cuts) (width 0.1))
 (gr_line (start 113.665 104.14) (end 113.665 64.77) (layer Edge.Cuts) (width 0.1))
 (gr_line (start 177.8 104.14) (end 99.06 104.14) (layer Edge.Cuts) (width 0.1))
 (segment (start 116.96 92.71) (end 116.96 99.695) (width 0.8) (layer B.Cu) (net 3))
 (segment (start 123.19 69.215) (end 123.19 71.755) (width 0.8) (layer B.Cu) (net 3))
 (segment (start 116.96 101.72) (end 116.96 99.695) (width 0.8) (layer B.Cu) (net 3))
 (segment (start 118.11 102.87) (end 116.96 101.72) (width 0.8) (layer B.Cu) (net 3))
 (segment (start 143.51 102.87) (end 118.11 102.87) (width 0.8) (layer B.Cu) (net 3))
 (segment (start 116.96 85.845) (end 116.84 85.725) (width 0.8) (layer B.Cu) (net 3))
 (segment (start 116.96 92.71) (end 116.96 85.845) (width 0.8) (layer B.Cu) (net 3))
 (segment (start 116.84 85.725) (end 116.84 83.185) (width 0.8) (layer B.Cu) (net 3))
 (segment (start 116.84 83.185) (end 116.84 80.645) (width 0.8) (layer B.Cu) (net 3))
 (segment (start 123.19 72.456507) (end 123.19 71.755) (width 0.8) (layer B.Cu) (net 3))
 (segment (start 116.84 78.806507) (end 123.19 72.456507) (width 0.8) (layer B.Cu) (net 3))
 (segment (start 116.84 80.645) (end 116.84 78.806507) (width 0.8) (layer B.Cu) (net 3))
 (segment (start 135.89 80.645) (end 137.16 79.375) (width 0.8) (layer B.Cu) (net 3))
 (segment (start 137.16 79.375) (end 139.7 79.375) (width 0.8) (layer B.Cu) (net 3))
 (segment (start 135.89 83.185) (end 135.89 80.645) (width 0.8) (layer B.Cu) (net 3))
 (segment (start 135.255 83.82) (end 135.89 83.185) (width 0.8) (layer B.Cu) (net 3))
 (segment (start 133.985 83.82) (end 135.255 83.82) (width 0.8) (layer B.Cu) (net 3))
 (segment (start 168.275 102.87) (end 143.51 102.87) (width 0.8) (layer B.Cu) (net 3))
 (segment (start 169.545 101.6) (end 168.275 102.87) (width 0.8) (layer B.Cu) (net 3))
 (segment (start 169.545 86.995) (end 169.545 101.6) (width 0.8) (layer B.Cu) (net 3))
 (segment (start 145.415 102.87) (end 143.51 102.87) (width 0.8) (layer B.Cu) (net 3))
 (segment (start 145.415 81.915) (end 145.415 102.87) (width 0.8) (layer B.Cu) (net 3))
 (segment (start 142.875 79.375) (end 145.415 81.915) (width 0.8) (layer B.Cu) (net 3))
 (segment (start 139.7 79.375) (end 142.875 79.375) (width 0.8) (layer B.Cu) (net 3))
 (segment (start 128.27 92.71) (end 130.175 94.615) (width 0.8) (layer B.Cu) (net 15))
 (segment (start 124.46 92.71) (end 128.27 92.71) (width 0.8) (layer B.Cu) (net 15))
 (segment (start 130.175 94.615) (end 132.715 94.615) (width 0.8) (layer B.Cu) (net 15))
 (segment (start 135.255 97.155) (end 139.7 97.155) (width 0.8) (layer B.Cu) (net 15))
 (segment (start 132.715 94.615) (end 135.255 97.155) (width 0.8) (layer B.Cu) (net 15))
 (segment (start 130.175 97.155) (end 130.175 99.695) (width 0.8) (layer B.Cu) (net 14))
 (segment (start 130.175 99.695) (end 139.7 99.695) (width 0.8) (layer B.Cu) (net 14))
 (segment (start 124.46 99.695) (end 130.175 99.695) (width 0.8) (layer B.Cu) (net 14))
 (segment (start 165.1 74.93) (end 165.1 72.39) (width 0.8) (layer B.Cu) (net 9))
 (segment (start 165.1 69.85) (end 165.1 72.39) (width 0.8) (layer B.Cu) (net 9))
 (segment (start 142.143482 66.009989) (end 121.315011 66.009989) (width 0.8) (layer B.Cu) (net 9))
 (segment (start 154.94 79.375) (end 152.4 79.375) (width 0.8) (layer B.Cu) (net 9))
 (segment (start 152.4 79.375) (end 146.685 73.66) (width 0.8) (layer B.Cu) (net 9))
 (segment (start 146.685 73.66) (end 146.685 70.551507) (width 0.8) (layer B.Cu) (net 9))
 (segment (start 121.315011 66.009989) (end 120.65 66.675) (width 0.8) (layer B.Cu) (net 9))
 (segment (start 146.685 70.551507) (end 142.143482 66.009989) (width 0.8) (layer B.Cu) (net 9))
 (segment (start 120.65 66.675) (end 120.65 71.755) (width 0.8) (layer B.Cu) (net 9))
 (segment (start 154.94 79.375) (end 158.355 79.375) (width 0.8) (layer B.Cu) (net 9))
 (segment (start 158.355 79.375) (end 162.8 74.93) (width 0.8) (layer B.Cu) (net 9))
 (segment (start 162.8 74.93) (end 165.1 74.93) (width 0.8) (layer B.Cu) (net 9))
 (segment (start 125.73 73.66) (end 125.73 71.755) (width 0.8) (layer B.Cu) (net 6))
 (segment (start 123.825 75.565) (end 125.73 73.66) (width 0.8) (layer B.Cu) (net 6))
 (segment (start 123.825 84.455) (end 123.825 75.565) (width 0.8) (layer B.Cu) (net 6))
 (segment (start 127 67.31) (end 125.73 68.58) (width 0.8) (layer B.Cu) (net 8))
 (segment (start 144.145 73.025) (end 144.145 69.85) (width 0.8) (layer B.Cu) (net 8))
 (segment (start 139.7 74.295) (end 142.875 74.295) (width 0.8) (layer B.Cu) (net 8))
 (segment (start 142.875 74.295) (end 144.145 73.025) (width 0.8) (layer B.Cu) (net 8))
 (segment (start 141.605 67.31) (end 127 67.31) (width 0.8) (layer B.Cu) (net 8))
 (segment (start 144.145 69.85) (end 141.605 67.31) (width 0.8) (layer B.Cu) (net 8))
 (segment (start 128.27 77.47) (end 129.54 78.74) (width 0.8) (layer B.Cu) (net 5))
 (segment (start 128.27 71.755) (end 128.27 77.47) (width 0.8) (layer B.Cu) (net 5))
 (segment (start 129.54 78.74) (end 133.985 78.74) (width 0.8) (layer B.Cu) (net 5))
 (segment (start 128.27 69.215) (end 132.715 69.215) (width 0.8) (layer B.Cu) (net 7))
 (segment (start 135.255 71.755) (end 139.7 71.755) (width 0.8) (layer B.Cu) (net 7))
 (segment (start 132.715 69.215) (end 135.255 71.755) (width 0.8) (layer B.Cu) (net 7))
 (segment (start 161.29 86.995) (end 154.94 86.995) (width 0.8) (layer B.Cu) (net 16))
 (segment (start 164.465 83.82) (end 161.29 86.995) (width 0.8) (layer B.Cu) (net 16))
 (segment (start 163.83 89.535) (end 154.94 89.535) (width 0.8) (layer B.Cu) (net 13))
 (segment (start 164.465 88.9) (end 163.83 89.535) (width 0.8) (layer B.Cu) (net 13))
 (segment (start 163.83 99.695) (end 154.94 99.695) (width 0.8) (layer B.Cu) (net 10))
 (segment (start 163.83 97.155) (end 154.94 97.155) (width 0.8) (layer B.Cu) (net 11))
 (segment (start 163.83 94.615) (end 154.94 94.615) (width 0.8) (layer B.Cu) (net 12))
 (segment (start 137.16 94.615) (end 139.7 94.615) (width 0.8) (layer B.Cu) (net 4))
 (segment (start 129.54 86.995) (end 137.16 94.615) (width 0.8) (layer B.Cu) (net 4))
 (segment (start 129.54 83.82) (end 129.54 86.995) (width 0.8) (layer B.Cu) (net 4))
 (segment (start 169.545 80.01) (end 169.545 84.455) (width 0.8) (layer B.Cu) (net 2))
 (segment (start 161.29 80.01) (end 164.465 80.01) (width 0.8) (layer B.Cu) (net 1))
 (segment (start 154.94 81.915) (end 159.385 81.915) (width 0.8) (layer B.Cu) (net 1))
 (segment (start 159.385 81.915) (end 161.29 80.01) (width 0.8) (layer B.Cu) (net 1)))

